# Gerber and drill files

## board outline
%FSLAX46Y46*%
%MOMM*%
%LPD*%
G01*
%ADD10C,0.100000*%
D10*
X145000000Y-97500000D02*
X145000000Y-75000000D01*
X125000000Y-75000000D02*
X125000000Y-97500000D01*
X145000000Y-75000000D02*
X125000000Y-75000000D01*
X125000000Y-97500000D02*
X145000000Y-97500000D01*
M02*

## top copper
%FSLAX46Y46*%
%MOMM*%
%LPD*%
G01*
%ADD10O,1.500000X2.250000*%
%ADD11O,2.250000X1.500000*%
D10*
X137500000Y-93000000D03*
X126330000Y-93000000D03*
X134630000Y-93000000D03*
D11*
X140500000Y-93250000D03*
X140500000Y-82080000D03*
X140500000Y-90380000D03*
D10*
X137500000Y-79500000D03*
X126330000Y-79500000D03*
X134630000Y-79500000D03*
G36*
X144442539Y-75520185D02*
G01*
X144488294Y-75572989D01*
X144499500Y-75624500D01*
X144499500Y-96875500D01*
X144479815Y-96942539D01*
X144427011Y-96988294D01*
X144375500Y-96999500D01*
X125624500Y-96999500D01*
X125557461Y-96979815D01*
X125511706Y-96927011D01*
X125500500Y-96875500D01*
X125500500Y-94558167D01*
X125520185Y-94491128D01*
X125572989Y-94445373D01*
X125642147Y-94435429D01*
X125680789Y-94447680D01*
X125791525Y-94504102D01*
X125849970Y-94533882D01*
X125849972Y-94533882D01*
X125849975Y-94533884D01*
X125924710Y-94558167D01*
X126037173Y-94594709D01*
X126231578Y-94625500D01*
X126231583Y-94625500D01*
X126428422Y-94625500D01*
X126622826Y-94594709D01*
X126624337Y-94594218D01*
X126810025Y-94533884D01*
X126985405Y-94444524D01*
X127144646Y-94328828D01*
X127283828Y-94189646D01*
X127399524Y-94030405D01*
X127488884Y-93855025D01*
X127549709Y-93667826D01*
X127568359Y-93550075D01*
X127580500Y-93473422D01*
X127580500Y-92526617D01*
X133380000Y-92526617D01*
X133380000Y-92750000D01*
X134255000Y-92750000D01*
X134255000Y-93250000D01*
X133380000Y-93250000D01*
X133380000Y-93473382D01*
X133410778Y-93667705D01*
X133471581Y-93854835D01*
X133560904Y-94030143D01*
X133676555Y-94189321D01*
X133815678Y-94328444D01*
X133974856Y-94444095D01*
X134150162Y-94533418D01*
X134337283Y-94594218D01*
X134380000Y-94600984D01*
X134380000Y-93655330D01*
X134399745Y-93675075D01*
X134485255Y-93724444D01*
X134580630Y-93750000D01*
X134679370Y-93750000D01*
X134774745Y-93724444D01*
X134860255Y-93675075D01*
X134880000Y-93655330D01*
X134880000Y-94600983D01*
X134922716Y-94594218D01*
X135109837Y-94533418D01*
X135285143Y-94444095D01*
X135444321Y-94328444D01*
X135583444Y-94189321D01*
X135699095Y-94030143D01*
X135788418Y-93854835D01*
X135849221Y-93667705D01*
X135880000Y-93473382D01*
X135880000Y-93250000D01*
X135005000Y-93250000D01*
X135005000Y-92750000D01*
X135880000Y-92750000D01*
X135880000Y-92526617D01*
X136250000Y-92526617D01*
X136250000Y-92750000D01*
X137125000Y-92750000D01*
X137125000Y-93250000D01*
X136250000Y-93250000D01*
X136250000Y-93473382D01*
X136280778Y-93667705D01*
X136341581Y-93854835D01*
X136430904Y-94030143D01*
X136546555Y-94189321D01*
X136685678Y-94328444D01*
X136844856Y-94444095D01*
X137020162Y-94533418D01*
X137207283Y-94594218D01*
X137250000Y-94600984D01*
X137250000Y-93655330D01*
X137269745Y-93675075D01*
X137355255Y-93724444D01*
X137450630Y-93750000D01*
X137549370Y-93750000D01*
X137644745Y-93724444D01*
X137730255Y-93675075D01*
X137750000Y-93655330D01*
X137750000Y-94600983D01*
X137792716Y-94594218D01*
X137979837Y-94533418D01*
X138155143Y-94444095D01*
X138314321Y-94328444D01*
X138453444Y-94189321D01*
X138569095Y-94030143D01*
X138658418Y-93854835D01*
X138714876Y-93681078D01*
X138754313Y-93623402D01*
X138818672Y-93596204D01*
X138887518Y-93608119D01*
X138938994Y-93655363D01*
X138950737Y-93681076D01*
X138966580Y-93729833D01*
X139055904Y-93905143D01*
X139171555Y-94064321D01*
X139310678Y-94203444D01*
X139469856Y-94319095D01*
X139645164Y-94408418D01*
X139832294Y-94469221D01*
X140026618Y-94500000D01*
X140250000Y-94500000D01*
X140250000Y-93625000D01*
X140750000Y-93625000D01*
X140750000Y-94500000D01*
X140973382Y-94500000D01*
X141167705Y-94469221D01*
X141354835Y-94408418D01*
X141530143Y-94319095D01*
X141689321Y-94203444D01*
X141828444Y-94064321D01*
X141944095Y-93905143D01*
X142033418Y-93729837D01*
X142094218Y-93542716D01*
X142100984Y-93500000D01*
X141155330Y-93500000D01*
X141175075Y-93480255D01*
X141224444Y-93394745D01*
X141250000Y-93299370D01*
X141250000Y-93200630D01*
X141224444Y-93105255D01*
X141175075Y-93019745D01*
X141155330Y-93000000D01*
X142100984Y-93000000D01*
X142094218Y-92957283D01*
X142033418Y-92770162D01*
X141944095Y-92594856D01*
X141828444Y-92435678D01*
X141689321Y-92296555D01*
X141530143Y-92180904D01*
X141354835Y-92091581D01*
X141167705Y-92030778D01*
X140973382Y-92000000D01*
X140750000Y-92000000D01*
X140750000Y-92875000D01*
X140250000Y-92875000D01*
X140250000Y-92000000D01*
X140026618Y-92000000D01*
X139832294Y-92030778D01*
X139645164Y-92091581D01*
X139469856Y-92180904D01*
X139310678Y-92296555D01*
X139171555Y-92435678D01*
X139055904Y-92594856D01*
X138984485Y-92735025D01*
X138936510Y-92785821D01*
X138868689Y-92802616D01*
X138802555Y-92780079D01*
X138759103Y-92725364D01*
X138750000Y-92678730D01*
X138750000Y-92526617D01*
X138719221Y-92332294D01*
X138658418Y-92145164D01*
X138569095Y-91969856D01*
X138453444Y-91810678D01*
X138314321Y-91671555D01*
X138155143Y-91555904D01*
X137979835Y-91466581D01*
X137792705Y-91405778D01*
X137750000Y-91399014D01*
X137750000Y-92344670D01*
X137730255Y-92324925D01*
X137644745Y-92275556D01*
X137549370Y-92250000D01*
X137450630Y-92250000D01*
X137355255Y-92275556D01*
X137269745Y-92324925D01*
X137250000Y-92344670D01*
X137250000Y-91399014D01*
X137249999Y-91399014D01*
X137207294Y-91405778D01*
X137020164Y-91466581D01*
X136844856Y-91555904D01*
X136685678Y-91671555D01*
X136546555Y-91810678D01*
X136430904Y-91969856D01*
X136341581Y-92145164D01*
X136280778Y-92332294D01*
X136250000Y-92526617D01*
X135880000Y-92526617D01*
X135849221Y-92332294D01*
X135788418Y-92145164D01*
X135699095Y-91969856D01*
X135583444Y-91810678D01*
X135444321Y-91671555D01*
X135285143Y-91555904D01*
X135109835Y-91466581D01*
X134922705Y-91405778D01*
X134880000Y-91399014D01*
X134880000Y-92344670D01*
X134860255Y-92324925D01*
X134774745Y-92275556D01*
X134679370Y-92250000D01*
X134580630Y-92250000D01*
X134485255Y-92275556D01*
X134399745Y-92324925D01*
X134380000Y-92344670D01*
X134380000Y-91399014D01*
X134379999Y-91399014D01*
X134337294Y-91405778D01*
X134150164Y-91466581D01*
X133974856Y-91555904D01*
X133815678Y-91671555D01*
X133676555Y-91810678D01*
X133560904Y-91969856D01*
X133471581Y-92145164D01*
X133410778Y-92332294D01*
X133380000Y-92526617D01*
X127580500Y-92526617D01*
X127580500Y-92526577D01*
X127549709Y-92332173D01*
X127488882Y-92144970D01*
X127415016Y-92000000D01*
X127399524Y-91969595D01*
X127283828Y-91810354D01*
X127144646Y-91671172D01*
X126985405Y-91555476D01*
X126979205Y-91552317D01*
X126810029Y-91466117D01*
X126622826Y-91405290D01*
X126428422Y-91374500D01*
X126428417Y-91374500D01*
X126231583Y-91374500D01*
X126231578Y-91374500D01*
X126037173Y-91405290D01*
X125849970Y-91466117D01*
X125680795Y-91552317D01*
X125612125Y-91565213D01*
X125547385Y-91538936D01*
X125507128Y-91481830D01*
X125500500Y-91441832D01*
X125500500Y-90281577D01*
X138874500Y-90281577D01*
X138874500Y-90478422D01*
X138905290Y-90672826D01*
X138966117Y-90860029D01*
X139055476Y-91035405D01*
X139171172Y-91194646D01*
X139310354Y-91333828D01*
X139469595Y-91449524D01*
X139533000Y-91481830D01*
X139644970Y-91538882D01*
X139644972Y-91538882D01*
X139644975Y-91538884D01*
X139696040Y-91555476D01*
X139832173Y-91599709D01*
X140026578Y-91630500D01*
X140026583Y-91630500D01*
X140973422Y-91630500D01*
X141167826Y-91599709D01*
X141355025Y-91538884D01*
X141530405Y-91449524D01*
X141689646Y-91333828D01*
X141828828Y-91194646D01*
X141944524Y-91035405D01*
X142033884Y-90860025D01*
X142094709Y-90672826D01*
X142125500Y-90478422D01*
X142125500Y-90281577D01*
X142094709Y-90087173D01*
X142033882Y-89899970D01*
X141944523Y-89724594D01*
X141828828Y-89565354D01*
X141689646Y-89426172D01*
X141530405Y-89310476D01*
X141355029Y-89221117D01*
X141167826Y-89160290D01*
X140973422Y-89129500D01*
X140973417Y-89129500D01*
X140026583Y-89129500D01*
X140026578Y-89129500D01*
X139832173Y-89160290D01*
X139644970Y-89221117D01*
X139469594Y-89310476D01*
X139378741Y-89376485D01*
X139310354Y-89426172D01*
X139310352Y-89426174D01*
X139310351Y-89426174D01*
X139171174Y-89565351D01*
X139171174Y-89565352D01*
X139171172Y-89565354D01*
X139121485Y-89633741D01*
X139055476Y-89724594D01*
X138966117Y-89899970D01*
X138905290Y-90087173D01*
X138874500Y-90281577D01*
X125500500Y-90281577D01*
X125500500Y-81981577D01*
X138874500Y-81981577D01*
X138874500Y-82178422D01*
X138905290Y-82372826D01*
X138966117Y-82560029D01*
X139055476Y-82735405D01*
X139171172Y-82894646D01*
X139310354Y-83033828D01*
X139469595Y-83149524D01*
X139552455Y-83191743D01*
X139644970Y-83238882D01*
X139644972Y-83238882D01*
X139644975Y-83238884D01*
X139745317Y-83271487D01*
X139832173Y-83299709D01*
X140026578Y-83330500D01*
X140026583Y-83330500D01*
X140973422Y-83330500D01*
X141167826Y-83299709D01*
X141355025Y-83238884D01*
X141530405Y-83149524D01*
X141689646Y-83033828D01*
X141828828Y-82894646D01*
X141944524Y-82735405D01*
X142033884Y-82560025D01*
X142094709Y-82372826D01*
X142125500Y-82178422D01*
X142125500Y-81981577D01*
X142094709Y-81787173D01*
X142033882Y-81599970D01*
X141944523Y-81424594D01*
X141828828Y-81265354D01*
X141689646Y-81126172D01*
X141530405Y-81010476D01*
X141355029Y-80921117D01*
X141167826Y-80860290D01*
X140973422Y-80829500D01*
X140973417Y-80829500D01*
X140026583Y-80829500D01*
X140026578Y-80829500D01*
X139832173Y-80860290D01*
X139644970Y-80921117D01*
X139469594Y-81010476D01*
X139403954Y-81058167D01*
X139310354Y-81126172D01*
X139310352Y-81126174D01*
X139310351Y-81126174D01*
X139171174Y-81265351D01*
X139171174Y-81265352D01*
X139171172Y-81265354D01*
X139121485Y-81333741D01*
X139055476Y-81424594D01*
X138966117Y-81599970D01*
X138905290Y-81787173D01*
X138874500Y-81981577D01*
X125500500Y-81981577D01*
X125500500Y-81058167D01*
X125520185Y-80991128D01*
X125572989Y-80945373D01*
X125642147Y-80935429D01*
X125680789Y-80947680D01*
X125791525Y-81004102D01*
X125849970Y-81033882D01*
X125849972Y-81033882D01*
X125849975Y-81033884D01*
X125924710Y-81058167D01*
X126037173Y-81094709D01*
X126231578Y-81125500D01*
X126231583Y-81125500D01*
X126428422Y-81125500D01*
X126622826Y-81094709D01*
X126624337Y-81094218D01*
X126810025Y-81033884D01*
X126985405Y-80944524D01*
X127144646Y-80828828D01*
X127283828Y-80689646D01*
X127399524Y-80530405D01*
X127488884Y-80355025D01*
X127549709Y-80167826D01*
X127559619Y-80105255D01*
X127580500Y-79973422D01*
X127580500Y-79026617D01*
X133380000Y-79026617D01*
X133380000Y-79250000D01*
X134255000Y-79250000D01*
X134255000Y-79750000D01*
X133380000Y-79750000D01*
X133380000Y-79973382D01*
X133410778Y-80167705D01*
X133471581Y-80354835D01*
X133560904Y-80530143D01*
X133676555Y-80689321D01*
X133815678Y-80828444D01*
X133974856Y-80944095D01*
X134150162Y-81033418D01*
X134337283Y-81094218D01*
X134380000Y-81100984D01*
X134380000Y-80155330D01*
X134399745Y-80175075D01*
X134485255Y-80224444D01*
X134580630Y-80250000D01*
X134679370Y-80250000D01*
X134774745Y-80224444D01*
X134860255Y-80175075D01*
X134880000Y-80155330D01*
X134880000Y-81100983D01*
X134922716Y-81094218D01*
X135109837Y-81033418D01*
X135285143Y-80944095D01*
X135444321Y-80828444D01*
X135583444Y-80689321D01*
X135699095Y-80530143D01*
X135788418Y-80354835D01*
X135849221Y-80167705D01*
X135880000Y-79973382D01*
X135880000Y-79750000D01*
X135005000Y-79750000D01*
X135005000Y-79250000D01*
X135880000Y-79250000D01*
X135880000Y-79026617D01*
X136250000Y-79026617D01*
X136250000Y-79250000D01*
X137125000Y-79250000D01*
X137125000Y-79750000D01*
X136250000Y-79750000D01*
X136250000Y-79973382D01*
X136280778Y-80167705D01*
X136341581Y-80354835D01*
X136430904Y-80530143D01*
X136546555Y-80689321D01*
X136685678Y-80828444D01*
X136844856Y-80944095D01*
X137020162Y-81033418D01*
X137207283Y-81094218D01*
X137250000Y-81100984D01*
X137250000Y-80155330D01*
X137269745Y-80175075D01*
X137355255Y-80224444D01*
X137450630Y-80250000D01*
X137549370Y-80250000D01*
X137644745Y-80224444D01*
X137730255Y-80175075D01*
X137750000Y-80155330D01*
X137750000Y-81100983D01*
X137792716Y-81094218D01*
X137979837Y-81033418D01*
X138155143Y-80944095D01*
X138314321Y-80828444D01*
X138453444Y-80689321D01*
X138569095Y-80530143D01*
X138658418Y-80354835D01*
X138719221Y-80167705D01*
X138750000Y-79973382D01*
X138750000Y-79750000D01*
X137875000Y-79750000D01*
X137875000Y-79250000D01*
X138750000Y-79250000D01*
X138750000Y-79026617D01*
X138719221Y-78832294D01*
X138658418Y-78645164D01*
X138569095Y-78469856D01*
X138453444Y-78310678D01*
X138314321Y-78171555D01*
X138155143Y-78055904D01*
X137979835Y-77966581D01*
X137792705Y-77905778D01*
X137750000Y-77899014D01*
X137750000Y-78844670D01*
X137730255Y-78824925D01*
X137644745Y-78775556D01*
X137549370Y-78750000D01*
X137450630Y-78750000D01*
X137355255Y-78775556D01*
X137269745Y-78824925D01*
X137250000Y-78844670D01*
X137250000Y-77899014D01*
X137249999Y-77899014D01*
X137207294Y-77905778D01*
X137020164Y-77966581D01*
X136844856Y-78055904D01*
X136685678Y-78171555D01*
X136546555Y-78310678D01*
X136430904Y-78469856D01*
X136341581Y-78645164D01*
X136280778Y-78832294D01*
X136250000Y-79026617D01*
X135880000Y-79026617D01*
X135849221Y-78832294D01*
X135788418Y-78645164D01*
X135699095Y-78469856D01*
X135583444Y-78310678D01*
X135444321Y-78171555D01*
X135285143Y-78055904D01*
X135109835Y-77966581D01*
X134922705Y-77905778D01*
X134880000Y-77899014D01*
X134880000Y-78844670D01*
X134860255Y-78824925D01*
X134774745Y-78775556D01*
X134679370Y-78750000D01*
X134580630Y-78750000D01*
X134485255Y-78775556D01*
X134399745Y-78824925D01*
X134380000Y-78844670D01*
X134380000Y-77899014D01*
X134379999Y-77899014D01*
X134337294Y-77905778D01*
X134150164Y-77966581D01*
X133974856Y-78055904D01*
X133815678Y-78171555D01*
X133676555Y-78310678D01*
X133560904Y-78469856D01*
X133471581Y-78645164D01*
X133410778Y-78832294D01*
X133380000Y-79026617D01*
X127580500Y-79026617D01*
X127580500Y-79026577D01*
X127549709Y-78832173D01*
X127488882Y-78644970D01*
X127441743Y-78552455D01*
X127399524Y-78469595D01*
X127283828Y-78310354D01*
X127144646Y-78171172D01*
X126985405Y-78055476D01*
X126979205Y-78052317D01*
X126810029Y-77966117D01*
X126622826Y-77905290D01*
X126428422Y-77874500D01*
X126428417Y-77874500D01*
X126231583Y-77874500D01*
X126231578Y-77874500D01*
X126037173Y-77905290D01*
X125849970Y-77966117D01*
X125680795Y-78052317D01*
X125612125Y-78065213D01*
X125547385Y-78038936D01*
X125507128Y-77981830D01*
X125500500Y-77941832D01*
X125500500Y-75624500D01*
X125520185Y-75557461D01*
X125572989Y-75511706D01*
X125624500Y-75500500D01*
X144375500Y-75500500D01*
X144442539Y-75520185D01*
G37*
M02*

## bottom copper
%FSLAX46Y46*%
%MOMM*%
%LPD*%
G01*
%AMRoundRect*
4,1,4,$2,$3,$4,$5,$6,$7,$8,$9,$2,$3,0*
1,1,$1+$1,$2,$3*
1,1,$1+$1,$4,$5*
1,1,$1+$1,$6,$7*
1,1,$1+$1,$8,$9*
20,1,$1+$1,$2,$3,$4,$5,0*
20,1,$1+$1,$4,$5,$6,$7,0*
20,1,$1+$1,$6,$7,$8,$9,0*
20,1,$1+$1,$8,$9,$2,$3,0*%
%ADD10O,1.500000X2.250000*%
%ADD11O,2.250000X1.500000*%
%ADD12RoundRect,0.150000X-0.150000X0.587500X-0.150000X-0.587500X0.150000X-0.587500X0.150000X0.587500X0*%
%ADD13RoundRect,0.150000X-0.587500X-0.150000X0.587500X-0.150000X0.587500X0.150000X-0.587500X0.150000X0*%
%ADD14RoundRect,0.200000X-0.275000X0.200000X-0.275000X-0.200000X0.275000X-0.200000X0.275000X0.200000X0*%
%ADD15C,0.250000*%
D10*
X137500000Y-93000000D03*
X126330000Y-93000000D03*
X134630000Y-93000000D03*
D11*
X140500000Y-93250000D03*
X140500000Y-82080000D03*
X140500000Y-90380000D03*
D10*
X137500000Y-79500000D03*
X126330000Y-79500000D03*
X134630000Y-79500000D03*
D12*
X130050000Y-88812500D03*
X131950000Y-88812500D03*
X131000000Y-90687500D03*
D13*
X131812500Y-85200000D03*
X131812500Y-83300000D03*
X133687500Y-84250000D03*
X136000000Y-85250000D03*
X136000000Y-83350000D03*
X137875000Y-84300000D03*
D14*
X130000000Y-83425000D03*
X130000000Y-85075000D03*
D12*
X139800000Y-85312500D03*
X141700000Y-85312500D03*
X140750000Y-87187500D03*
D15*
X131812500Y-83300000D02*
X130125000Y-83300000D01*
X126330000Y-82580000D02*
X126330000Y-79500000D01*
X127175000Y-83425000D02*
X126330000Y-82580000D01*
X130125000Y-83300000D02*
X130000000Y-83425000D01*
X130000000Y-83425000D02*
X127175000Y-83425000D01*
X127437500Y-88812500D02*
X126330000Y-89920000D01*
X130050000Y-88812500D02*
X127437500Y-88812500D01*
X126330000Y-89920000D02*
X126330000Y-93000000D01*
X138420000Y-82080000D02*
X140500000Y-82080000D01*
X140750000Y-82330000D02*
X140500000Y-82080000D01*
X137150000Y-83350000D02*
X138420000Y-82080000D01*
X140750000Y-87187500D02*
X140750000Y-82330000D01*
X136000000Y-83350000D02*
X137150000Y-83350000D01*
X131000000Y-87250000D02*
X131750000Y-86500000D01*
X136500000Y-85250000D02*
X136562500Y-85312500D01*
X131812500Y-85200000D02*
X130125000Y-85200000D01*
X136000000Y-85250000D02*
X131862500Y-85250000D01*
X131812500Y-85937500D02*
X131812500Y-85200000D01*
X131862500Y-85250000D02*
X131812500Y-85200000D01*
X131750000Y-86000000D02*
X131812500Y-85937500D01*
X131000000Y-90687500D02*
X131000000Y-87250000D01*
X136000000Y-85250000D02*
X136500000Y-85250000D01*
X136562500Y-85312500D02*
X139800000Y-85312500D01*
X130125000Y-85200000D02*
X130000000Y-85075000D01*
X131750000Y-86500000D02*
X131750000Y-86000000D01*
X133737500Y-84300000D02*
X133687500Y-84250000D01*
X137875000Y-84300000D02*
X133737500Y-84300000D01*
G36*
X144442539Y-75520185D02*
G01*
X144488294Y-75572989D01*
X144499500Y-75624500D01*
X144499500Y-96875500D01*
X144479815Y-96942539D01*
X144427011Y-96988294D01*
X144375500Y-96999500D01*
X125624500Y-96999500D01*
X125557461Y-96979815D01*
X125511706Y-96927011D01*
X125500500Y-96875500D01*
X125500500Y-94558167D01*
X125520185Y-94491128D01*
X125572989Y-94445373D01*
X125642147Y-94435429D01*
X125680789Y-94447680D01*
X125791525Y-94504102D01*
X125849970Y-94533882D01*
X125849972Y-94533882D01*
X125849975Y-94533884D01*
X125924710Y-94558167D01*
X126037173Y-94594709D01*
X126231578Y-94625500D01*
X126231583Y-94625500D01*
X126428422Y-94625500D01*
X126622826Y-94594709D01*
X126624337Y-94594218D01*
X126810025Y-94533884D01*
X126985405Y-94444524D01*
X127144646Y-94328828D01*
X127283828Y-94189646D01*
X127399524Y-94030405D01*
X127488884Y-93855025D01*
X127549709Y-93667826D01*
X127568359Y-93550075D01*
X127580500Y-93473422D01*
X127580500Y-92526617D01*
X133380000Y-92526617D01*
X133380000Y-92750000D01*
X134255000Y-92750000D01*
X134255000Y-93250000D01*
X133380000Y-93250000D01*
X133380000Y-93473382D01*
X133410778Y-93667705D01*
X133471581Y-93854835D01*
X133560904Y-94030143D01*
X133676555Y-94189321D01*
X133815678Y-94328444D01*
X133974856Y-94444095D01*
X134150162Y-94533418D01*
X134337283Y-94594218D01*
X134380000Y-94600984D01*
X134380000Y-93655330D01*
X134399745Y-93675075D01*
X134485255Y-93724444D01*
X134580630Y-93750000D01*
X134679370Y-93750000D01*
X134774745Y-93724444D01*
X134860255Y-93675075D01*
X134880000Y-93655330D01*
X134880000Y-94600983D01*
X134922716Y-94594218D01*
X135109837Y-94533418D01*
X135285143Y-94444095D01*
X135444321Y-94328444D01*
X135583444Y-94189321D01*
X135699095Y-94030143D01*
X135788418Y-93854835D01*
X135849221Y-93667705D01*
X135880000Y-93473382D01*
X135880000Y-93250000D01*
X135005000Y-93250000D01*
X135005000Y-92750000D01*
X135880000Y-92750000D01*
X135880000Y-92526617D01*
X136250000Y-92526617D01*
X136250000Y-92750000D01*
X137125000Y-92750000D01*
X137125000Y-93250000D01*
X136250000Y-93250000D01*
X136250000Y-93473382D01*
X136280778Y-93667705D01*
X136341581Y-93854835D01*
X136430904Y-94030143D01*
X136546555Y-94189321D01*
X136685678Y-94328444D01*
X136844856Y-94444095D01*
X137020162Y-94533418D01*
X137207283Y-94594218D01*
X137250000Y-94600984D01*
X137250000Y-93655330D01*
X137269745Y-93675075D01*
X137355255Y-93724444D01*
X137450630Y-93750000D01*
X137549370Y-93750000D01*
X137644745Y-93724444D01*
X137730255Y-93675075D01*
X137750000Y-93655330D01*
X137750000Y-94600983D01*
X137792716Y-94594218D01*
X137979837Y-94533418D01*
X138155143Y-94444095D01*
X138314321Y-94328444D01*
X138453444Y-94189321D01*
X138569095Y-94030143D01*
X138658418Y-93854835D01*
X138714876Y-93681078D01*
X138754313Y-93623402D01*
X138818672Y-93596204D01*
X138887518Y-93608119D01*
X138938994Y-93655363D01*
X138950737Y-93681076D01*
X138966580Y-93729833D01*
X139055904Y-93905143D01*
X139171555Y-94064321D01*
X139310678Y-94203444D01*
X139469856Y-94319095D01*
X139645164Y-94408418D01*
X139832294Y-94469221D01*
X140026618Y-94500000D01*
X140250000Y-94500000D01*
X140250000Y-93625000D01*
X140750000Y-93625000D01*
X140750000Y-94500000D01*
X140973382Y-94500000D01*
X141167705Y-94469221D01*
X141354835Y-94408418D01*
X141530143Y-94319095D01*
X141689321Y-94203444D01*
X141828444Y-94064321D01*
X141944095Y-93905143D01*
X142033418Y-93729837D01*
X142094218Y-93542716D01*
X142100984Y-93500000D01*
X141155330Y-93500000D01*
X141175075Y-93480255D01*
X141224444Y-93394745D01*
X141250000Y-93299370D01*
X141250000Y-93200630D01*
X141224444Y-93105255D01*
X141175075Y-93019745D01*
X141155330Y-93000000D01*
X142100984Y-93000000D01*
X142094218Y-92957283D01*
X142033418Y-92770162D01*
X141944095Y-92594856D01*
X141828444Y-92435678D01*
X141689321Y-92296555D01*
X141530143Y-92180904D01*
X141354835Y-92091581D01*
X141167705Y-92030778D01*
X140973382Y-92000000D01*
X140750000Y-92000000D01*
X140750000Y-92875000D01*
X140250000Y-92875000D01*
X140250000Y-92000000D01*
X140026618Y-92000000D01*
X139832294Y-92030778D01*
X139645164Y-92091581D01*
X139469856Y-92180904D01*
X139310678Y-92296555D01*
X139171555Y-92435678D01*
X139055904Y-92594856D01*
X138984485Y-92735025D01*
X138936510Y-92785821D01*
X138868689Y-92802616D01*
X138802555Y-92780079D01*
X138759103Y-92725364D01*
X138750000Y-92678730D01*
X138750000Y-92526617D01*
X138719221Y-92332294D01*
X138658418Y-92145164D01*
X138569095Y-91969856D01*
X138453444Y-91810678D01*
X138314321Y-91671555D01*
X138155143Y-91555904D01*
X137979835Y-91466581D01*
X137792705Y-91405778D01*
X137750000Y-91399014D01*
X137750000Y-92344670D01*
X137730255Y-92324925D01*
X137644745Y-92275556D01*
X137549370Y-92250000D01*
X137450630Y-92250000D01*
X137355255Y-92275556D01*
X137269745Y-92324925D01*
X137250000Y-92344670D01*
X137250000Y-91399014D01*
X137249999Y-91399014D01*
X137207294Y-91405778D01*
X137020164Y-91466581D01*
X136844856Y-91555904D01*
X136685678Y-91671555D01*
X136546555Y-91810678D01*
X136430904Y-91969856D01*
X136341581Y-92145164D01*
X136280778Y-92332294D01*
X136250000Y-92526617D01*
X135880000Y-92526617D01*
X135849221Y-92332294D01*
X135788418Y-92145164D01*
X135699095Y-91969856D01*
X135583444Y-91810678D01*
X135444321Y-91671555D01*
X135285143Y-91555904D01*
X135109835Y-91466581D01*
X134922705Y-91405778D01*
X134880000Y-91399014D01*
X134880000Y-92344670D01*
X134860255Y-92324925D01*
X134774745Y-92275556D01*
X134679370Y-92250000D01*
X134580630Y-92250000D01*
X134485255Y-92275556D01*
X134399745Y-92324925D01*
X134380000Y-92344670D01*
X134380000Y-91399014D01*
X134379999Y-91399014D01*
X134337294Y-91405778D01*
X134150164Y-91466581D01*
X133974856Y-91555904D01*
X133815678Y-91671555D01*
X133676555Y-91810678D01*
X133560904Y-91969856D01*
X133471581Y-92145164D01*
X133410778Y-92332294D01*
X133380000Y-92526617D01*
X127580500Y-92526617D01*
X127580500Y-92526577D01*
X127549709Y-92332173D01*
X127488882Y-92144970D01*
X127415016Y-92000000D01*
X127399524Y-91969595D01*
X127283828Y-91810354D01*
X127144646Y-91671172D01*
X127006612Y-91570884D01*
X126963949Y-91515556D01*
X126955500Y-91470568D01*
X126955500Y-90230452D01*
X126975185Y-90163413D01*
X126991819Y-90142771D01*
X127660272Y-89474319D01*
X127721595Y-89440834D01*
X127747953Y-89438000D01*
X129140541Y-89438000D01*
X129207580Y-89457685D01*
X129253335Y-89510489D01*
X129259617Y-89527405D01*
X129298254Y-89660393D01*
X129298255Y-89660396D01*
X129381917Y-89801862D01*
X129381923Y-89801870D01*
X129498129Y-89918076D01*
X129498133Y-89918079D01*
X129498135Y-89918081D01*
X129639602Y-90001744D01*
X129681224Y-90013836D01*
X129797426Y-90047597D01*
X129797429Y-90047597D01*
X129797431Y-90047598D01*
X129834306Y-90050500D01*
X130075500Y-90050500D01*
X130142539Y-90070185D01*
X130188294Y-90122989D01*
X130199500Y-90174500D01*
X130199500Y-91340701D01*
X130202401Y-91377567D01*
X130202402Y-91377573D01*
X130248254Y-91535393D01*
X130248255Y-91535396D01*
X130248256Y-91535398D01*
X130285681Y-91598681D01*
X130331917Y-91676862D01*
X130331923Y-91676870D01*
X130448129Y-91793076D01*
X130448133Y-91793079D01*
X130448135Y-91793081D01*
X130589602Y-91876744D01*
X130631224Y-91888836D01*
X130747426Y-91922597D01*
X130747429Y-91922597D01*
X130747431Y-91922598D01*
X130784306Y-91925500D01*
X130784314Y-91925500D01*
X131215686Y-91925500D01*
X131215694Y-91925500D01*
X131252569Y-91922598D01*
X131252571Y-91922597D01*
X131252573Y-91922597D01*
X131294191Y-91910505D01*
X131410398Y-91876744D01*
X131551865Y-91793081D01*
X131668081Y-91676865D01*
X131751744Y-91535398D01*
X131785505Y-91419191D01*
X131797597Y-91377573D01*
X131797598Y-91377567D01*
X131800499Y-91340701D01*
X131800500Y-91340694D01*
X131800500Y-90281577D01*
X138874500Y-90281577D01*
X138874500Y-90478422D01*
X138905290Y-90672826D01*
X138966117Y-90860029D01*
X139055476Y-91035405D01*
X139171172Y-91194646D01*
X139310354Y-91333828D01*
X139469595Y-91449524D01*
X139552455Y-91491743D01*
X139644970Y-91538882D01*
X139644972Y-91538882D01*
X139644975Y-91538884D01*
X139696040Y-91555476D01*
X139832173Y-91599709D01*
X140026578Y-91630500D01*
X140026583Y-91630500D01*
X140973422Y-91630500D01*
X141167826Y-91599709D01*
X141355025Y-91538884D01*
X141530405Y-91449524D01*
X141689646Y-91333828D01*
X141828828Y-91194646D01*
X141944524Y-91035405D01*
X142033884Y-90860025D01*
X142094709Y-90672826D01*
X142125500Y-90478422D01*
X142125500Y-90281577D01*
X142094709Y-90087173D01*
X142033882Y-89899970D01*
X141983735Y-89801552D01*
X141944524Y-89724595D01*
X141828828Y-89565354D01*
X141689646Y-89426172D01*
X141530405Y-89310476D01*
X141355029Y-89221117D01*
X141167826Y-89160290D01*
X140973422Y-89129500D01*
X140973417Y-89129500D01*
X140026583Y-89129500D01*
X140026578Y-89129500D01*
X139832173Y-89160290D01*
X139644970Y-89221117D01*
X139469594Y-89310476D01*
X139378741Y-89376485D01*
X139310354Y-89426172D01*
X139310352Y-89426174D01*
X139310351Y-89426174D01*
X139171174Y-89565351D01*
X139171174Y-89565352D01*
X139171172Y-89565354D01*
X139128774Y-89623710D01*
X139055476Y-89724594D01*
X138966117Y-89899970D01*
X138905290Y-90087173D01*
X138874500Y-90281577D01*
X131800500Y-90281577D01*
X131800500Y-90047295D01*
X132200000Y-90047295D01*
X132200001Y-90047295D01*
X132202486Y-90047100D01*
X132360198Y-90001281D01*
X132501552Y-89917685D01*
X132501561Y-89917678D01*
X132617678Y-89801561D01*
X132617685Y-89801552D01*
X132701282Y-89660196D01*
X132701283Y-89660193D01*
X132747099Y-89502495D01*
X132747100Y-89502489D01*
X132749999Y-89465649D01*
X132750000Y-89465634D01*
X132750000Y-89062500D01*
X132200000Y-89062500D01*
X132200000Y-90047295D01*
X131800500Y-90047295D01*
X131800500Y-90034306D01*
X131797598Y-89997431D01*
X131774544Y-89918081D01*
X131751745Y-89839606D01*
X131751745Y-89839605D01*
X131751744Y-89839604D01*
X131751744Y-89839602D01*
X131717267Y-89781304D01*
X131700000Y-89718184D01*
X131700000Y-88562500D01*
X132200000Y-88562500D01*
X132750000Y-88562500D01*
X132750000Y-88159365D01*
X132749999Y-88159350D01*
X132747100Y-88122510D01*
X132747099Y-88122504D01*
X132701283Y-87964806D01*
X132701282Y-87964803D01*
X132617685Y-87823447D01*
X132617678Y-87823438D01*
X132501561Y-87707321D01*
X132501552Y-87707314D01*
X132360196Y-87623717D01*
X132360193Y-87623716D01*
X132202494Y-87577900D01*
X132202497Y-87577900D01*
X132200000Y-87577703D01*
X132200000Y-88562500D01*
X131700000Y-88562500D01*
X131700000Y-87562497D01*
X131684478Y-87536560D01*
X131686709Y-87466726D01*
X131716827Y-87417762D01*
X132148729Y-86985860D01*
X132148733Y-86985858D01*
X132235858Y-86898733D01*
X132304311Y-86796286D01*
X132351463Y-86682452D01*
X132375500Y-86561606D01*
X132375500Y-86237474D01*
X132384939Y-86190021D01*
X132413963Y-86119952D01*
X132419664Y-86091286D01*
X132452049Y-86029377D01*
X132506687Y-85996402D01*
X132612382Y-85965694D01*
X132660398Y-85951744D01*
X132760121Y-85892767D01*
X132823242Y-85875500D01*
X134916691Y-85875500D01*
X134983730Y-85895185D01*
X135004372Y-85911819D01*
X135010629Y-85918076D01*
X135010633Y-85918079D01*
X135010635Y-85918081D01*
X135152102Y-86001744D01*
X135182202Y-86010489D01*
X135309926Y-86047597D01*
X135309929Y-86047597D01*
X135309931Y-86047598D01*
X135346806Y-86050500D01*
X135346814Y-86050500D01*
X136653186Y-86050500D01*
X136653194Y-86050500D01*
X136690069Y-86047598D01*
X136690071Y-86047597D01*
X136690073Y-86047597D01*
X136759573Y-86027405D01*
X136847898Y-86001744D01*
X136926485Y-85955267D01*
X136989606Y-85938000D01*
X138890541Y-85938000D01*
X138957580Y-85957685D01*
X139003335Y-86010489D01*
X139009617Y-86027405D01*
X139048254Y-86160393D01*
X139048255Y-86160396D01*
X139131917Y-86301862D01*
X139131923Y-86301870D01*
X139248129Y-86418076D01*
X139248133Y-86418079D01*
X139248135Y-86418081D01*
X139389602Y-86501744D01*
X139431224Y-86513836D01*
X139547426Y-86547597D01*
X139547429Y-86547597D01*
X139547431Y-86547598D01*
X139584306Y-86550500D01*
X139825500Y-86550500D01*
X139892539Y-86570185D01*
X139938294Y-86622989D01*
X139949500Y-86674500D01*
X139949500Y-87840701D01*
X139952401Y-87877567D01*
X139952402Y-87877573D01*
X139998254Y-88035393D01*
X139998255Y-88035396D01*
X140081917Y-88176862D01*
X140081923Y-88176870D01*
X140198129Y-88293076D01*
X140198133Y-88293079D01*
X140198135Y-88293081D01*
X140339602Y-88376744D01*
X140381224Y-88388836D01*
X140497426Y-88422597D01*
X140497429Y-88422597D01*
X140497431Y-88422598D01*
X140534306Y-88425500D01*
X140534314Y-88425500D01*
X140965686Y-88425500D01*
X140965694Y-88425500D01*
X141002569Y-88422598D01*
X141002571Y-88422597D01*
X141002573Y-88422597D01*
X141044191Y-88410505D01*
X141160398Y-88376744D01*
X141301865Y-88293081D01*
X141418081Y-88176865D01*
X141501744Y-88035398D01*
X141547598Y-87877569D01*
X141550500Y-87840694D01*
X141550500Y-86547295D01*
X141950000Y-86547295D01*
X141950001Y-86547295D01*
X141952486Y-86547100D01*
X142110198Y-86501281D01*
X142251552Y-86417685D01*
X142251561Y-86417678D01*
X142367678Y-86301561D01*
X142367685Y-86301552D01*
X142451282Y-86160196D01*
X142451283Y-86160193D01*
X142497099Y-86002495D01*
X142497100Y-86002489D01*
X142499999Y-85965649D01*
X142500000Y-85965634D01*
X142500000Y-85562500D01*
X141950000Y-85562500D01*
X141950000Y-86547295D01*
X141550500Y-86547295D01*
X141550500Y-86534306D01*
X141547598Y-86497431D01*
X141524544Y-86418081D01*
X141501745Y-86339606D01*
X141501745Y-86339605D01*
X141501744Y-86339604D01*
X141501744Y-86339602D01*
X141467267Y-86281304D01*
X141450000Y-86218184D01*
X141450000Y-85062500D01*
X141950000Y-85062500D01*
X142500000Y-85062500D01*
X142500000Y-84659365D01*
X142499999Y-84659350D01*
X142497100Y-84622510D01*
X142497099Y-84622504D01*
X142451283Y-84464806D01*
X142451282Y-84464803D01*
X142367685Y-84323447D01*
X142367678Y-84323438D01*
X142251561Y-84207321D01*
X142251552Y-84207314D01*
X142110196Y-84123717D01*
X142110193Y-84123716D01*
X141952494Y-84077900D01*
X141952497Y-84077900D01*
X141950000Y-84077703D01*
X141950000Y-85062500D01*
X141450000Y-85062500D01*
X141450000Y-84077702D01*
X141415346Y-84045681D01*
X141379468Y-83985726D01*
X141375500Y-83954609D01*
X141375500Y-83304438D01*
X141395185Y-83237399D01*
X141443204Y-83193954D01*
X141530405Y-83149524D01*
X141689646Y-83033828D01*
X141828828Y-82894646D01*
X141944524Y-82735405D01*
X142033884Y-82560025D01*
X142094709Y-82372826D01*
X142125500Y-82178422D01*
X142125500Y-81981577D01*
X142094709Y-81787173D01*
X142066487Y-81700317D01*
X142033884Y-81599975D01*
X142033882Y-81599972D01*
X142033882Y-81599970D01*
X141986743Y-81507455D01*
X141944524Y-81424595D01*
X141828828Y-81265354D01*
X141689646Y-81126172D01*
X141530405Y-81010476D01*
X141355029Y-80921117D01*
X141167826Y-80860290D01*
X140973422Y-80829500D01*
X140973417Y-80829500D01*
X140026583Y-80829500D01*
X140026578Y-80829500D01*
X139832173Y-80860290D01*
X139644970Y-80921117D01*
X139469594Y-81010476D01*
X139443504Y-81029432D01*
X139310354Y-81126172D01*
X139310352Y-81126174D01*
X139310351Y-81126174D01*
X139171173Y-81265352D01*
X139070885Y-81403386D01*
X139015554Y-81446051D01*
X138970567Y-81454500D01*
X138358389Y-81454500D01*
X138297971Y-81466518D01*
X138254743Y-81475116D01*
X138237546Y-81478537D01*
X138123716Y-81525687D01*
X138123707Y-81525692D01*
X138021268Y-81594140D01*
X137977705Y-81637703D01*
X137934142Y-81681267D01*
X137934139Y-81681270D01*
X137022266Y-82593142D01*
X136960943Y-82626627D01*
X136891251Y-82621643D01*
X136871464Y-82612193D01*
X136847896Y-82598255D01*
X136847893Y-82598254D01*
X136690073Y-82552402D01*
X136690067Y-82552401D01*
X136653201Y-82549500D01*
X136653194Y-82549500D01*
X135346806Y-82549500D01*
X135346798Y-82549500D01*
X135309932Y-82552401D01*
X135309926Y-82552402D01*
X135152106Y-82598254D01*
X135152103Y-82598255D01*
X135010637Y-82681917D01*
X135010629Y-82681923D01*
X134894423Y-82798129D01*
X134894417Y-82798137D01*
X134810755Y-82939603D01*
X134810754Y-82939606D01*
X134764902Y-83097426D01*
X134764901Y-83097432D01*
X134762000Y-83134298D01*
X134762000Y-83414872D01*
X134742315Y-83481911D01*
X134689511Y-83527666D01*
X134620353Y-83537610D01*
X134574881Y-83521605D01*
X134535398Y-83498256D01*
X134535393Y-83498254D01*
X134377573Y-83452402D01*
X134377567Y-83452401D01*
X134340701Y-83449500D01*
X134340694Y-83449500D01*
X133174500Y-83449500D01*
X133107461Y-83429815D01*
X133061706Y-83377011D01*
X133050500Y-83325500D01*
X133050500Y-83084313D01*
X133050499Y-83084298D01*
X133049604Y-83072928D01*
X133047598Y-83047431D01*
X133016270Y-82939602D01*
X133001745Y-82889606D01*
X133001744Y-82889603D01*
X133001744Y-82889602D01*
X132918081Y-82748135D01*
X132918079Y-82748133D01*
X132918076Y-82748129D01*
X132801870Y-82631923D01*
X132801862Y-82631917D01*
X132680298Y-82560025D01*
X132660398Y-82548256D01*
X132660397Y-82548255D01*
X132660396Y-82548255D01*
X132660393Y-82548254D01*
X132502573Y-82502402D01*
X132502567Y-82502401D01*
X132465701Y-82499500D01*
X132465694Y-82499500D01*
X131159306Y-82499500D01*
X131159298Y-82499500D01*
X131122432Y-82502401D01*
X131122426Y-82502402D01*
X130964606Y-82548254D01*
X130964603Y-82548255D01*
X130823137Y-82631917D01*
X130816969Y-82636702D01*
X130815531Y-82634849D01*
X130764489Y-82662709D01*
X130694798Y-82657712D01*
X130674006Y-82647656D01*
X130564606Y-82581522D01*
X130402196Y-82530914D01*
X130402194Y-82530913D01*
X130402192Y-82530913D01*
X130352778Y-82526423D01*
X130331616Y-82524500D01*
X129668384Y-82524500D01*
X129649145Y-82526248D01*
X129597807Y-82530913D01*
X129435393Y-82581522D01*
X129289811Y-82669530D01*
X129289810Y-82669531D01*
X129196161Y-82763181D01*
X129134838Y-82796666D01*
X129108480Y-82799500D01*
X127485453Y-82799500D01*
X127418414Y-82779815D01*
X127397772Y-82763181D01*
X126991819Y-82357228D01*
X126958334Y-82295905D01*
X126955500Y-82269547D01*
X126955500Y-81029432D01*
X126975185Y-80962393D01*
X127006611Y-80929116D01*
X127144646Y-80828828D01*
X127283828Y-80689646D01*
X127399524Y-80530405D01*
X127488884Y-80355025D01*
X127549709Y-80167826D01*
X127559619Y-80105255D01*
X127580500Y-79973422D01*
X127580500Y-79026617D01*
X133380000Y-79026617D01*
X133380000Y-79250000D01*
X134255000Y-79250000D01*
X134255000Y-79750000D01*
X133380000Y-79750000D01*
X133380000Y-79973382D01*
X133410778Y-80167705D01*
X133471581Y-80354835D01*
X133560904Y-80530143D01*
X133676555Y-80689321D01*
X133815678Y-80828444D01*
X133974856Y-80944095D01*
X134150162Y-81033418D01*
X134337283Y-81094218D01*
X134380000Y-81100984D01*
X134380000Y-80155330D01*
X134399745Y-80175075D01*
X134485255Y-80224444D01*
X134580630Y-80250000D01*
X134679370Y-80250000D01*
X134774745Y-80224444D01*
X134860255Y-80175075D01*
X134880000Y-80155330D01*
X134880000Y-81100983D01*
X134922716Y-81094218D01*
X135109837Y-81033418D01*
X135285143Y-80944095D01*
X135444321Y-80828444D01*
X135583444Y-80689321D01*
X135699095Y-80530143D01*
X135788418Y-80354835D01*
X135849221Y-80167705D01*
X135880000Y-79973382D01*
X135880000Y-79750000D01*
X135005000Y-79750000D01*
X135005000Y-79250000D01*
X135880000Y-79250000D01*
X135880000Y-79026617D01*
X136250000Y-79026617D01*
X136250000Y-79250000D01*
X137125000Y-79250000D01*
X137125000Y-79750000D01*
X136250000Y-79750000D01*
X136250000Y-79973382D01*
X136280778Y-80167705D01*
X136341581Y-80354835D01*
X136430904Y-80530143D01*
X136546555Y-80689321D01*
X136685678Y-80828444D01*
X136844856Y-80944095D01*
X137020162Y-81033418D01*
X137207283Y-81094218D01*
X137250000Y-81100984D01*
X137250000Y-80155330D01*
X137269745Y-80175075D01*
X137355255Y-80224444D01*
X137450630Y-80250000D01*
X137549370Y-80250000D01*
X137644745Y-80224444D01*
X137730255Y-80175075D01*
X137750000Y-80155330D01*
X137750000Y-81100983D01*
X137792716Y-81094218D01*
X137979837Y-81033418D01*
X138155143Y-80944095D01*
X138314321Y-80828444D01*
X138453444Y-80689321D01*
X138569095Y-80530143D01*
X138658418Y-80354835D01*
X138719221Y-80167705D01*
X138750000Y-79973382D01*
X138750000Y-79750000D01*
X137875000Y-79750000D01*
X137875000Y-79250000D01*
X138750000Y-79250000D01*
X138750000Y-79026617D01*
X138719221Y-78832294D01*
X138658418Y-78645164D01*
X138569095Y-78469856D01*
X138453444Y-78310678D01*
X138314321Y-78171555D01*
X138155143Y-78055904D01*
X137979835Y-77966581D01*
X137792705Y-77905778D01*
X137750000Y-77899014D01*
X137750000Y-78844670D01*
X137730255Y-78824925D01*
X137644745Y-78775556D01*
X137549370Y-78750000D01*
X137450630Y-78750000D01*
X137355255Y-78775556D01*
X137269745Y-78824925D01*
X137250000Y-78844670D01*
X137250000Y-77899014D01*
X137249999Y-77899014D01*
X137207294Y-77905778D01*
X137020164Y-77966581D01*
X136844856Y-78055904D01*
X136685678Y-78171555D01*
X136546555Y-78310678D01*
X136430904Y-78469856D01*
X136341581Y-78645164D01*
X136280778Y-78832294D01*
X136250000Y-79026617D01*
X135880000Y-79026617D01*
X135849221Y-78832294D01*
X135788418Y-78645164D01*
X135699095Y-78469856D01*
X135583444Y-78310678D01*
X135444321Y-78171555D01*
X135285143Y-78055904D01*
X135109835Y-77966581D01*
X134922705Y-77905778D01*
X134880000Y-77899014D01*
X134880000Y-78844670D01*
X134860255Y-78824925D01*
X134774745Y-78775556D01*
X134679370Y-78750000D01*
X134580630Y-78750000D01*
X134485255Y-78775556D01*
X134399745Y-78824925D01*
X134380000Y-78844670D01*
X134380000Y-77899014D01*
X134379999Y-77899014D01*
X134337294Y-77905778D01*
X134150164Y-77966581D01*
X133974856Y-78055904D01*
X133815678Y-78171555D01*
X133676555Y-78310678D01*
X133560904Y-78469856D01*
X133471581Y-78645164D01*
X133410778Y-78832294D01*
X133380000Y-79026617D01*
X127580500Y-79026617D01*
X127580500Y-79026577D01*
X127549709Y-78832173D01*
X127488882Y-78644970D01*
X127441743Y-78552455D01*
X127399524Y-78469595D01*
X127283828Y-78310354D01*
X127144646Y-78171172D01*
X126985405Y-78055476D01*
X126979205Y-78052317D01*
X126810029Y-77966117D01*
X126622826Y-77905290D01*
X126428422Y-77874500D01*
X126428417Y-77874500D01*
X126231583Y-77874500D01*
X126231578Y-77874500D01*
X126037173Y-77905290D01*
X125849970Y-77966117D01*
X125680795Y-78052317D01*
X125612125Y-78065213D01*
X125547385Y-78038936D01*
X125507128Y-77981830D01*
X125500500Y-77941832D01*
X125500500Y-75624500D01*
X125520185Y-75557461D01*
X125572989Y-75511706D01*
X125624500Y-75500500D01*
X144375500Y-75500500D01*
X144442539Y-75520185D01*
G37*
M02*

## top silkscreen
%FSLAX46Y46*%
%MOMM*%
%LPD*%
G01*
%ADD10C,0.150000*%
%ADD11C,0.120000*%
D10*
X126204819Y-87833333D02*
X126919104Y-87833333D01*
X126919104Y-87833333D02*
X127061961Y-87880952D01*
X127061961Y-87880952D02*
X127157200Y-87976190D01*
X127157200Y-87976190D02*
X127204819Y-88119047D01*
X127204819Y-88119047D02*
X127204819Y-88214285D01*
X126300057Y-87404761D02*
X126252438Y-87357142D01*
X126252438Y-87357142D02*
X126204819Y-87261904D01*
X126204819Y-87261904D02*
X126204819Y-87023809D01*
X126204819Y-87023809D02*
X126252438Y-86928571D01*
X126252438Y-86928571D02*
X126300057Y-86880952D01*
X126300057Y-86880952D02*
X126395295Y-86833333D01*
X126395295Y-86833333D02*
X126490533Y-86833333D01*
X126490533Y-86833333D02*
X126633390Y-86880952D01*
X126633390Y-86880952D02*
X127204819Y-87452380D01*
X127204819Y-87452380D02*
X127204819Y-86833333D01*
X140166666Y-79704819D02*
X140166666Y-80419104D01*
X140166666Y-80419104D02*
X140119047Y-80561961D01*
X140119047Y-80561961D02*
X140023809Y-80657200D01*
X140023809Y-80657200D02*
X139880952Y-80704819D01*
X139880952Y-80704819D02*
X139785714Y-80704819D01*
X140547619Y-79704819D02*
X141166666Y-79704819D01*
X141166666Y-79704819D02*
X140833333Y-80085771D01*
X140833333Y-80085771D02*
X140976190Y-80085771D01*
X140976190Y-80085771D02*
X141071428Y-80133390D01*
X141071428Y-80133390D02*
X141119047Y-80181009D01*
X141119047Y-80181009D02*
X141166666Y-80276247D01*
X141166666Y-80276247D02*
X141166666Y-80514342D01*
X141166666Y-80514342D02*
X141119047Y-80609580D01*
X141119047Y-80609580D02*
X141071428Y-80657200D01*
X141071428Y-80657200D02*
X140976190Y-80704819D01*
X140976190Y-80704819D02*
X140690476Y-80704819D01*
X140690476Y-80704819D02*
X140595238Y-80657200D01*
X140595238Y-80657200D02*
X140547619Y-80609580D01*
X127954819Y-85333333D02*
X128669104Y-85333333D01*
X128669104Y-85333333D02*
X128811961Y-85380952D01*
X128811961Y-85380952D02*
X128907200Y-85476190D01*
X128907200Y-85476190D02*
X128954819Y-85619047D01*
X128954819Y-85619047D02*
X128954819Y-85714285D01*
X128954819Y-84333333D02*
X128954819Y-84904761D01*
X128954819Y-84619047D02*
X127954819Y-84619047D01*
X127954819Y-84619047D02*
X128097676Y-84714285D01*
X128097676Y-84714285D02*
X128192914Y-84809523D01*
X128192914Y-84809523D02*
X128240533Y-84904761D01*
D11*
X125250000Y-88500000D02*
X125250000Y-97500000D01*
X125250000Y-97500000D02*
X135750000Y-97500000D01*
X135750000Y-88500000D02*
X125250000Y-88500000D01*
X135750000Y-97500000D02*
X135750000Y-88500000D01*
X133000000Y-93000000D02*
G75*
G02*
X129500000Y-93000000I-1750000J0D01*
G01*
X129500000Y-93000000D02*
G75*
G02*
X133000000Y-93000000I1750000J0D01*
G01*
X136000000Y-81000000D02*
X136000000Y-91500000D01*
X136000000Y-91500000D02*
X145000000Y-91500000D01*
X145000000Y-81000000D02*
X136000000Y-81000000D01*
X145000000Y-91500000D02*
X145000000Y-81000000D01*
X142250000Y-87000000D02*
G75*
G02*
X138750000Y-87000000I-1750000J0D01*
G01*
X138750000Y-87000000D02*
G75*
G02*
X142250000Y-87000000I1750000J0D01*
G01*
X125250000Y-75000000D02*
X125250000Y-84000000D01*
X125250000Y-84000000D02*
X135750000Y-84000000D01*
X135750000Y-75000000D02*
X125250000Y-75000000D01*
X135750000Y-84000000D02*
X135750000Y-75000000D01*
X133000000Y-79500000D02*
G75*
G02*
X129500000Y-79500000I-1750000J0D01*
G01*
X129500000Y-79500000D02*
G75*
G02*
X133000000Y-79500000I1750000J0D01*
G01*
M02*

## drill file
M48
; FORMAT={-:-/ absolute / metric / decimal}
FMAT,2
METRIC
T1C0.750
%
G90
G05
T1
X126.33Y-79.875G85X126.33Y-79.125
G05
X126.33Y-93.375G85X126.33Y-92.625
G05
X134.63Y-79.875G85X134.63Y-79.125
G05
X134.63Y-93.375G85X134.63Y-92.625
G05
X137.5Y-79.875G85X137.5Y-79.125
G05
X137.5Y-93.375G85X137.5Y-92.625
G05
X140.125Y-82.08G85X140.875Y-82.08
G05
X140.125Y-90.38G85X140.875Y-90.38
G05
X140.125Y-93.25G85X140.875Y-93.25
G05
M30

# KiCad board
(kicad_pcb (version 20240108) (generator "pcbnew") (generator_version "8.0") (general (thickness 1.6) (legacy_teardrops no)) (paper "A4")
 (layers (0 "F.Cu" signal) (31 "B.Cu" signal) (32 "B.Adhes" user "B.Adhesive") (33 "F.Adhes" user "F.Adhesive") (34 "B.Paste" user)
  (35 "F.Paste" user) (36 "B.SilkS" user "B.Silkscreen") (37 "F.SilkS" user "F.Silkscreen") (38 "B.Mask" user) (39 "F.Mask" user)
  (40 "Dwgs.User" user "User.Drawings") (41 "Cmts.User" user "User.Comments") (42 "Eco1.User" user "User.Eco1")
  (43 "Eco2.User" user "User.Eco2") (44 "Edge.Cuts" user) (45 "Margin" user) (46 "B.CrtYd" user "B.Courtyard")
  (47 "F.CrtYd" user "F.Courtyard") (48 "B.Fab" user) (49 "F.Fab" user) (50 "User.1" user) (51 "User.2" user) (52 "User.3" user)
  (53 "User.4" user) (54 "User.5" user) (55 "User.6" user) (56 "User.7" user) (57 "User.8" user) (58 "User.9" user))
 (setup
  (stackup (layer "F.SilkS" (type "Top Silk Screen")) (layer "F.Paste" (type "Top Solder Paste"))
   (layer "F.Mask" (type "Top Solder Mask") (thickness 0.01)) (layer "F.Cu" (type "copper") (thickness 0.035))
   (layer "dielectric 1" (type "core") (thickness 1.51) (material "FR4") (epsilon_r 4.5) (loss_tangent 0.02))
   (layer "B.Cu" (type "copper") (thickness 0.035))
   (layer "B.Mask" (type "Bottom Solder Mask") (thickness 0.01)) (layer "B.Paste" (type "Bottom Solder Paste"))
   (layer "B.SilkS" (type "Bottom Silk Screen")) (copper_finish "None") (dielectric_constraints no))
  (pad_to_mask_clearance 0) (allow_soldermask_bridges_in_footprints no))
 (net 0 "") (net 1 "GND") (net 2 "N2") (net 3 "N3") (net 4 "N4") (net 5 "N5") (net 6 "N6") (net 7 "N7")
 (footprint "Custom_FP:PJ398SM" (layer "F.Cu") (at 131.25 93 90)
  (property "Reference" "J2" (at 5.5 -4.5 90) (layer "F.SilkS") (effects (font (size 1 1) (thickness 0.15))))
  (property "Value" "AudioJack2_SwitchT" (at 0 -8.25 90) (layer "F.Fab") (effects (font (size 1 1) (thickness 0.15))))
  (fp_line (start 4.5 -6) (end -4.5 -6) (stroke (width 0.12) (type solid)) (layer "F.SilkS"))
  (fp_line (start -4.5 -6) (end -4.5 4.5) (stroke (width 0.12) (type solid)) (layer "F.SilkS"))
  (fp_line (start 4.5 4.5) (end 4.5 -6) (stroke (width 0.12) (type solid)) (layer "F.SilkS"))
  (fp_line (start -4.5 4.5) (end 4.5 4.5) (stroke (width 0.12) (type solid)) (layer "F.SilkS"))
  (fp_circle (center 0 0) (end 1.75 0) (stroke (width 0.12) (type solid)) (fill none) (layer "F.SilkS"))
  (pad "S" thru_hole oval (at 0 6.25 90) (size 2.25 1.5) (drill oval 1.5 0.75) (layers "*.Cu" "*.Mask") (remove_unused_layers no)
   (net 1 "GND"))
  (pad "T" thru_hole oval (at 0 -4.92 90) (size 2.25 1.5) (drill oval 1.5 0.75) (layers "*.Cu" "*.Mask") (remove_unused_layers no)
   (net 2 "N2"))
  (pad "TN" thru_hole oval (at 0 3.38 90) (size 2.25 1.5) (drill oval 1.5 0.75) (layers "*.Cu" "*.Mask") (remove_unused_layers no)
   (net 1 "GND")))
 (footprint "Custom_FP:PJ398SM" (layer "F.Cu") (at 140.5 87)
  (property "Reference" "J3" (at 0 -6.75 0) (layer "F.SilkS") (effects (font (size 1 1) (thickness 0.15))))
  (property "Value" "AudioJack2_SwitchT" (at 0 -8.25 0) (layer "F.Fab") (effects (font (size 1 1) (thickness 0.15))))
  (fp_line (start -4.5 -6) (end -4.5 4.5) (stroke (width 0.12) (type solid)) (layer "F.SilkS"))
  (fp_line (start -4.5 4.5) (end 4.5 4.5) (stroke (width 0.12) (type solid)) (layer "F.SilkS"))
  (fp_line (start 4.5 -6) (end -4.5 -6) (stroke (width 0.12) (type solid)) (layer "F.SilkS"))
  (fp_line (start 4.5 4.5) (end 4.5 -6) (stroke (width 0.12) (type solid)) (layer "F.SilkS"))
  (fp_circle (center 0 0) (end 1.75 0) (stroke (width 0.12) (type solid)) (fill none) (layer "F.SilkS"))
  (pad "S" thru_hole oval (at 0 6.25) (size 2.25 1.5) (drill oval 1.5 0.75) (layers "*.Cu" "*.Mask") (remove_unused_layers no) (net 1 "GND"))
  (pad "T" thru_hole oval (at 0 -4.92) (size 2.25 1.5) (drill oval 1.5 0.75) (layers "*.Cu" "*.Mask") (remove_unused_layers no) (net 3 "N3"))
  (pad "TN" thru_hole oval (at 0 3.38) (size 2.25 1.5) (drill oval 1.5 0.75) (layers "*.Cu" "*.Mask") (remove_unused_layers no) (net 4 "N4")))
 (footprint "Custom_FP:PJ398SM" (layer "F.Cu") (at 131.25 79.5 90)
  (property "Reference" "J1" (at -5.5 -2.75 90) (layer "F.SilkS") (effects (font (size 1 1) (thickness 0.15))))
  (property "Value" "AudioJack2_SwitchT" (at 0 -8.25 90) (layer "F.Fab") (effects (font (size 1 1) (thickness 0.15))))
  (fp_line (start 4.5 -6) (end -4.5 -6) (stroke (width 0.12) (type solid)) (layer "F.SilkS"))
  (fp_line (start -4.5 -6) (end -4.5 4.5) (stroke (width 0.12) (type solid)) (layer "F.SilkS"))
  (fp_line (start 4.5 4.5) (end 4.5 -6) (stroke (width 0.12) (type solid)) (layer "F.SilkS"))
  (fp_line (start -4.5 4.5) (end 4.5 4.5) (stroke (width 0.12) (type solid)) (layer "F.SilkS"))
  (fp_circle (center 0 0) (end 1.75 0) (stroke (width 0.12) (type solid)) (fill none) (layer "F.SilkS"))
  (pad "S" thru_hole oval (at 0 6.25 90) (size 2.25 1.5) (drill oval 1.5 0.75) (layers "*.Cu" "*.Mask") (remove_unused_layers no)
   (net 1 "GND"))
  (pad "T" thru_hole oval (at 0 -4.92 90) (size 2.25 1.5) (drill oval 1.5 0.75) (layers "*.Cu" "*.Mask") (remove_unused_layers no)
   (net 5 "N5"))
  (pad "TN" thru_hole oval (at 0 3.38 90) (size 2.25 1.5) (drill oval 1.5 0.75) (layers "*.Cu" "*.Mask") (remove_unused_layers no)
   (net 1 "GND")))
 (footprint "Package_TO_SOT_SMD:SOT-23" (layer "B.Cu") (at 131 89.75 -90)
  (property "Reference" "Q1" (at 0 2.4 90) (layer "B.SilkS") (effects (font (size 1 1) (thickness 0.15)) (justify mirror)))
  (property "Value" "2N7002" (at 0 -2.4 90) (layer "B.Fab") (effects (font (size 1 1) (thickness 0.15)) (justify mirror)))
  (pad "1" smd roundrect (at -0.9375 0.95 270) (size 1.475 0.6) (layers "B.Cu" "B.Paste" "B.Mask") (roundrect_rratio 0.25) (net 2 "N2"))
  (pad "2" smd roundrect (at -0.9375 -0.95 270) (size 1.475 0.6) (layers "B.Cu" "B.Paste" "B.Mask") (roundrect_rratio 0.25) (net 1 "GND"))
  (pad "3" smd roundrect (at 0.9375 0 270) (size 1.475 0.6) (layers "B.Cu" "B.Paste" "B.Mask") (roundrect_rratio 0.25) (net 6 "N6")))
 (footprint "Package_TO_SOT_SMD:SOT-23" (layer "B.Cu") (at 132.75 84.25)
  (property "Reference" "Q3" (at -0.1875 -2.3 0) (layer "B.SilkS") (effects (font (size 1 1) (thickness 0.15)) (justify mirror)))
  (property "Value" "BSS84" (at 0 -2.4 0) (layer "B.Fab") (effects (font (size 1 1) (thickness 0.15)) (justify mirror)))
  (pad "1" smd roundrect (at -0.9375 0.95) (size 1.475 0.6) (layers "B.Cu" "B.Paste" "B.Mask") (roundrect_rratio 0.25) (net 6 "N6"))
  (pad "2" smd roundrect (at -0.9375 -0.95) (size 1.475 0.6) (layers "B.Cu" "B.Paste" "B.Mask") (roundrect_rratio 0.25) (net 5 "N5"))
  (pad "3" smd roundrect (at 0.9375 0) (size 1.475 0.6) (layers "B.Cu" "B.Paste" "B.Mask") (roundrect_rratio 0.25) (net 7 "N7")))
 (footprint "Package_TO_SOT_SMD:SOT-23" (layer "B.Cu") (at 136.9375 84.3)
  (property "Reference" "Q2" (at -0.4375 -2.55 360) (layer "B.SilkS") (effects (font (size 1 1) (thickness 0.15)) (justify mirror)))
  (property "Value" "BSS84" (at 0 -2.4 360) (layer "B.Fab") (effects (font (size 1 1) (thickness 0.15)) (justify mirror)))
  (pad "1" smd roundrect (at -0.9375 0.95) (size 1.475 0.6) (layers "B.Cu" "B.Paste" "B.Mask") (roundrect_rratio 0.25) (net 6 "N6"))
  (pad "2" smd roundrect (at -0.9375 -0.95) (size 1.475 0.6) (layers "B.Cu" "B.Paste" "B.Mask") (roundrect_rratio 0.25) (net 3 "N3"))
  (pad "3" smd roundrect (at 0.9375 0) (size 1.475 0.6) (layers "B.Cu" "B.Paste" "B.Mask") (roundrect_rratio 0.25) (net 7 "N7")))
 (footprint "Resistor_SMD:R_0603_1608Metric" (layer "B.Cu") (at 130 84.25 -90)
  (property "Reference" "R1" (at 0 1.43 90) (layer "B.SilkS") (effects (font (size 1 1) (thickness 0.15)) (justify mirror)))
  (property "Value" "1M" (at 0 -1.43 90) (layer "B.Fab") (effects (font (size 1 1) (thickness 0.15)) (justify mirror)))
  (pad "1" smd roundrect (at -0.825 0 270) (size 0.8 0.95) (layers "B.Cu" "B.Paste" "B.Mask") (roundrect_rratio 0.25) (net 5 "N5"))
  (pad "2" smd roundrect (at 0.825 0 270) (size 0.8 0.95) (layers "B.Cu" "B.Paste" "B.Mask") (roundrect_rratio 0.25) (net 6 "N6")))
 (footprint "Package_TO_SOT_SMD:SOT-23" (layer "B.Cu") (at 140.75 86.25 -90)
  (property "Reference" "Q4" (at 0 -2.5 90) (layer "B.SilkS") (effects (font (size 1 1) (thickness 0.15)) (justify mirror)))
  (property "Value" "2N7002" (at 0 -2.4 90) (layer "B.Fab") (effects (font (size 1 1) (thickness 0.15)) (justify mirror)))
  (pad "1" smd roundrect (at -0.9375 0.95 270) (size 1.475 0.6) (layers "B.Cu" "B.Paste" "B.Mask") (roundrect_rratio 0.25) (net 6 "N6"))
  (pad "2" smd roundrect (at -0.9375 -0.95 270) (size 1.475 0.6) (layers "B.Cu" "B.Paste" "B.Mask") (roundrect_rratio 0.25) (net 1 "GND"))
  (pad "3" smd roundrect (at 0.9375 0 270) (size 1.475 0.6) (layers "B.Cu" "B.Paste" "B.Mask") (roundrect_rratio 0.25) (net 3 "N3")))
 (gr_line (start 145 97.5) (end 145 75) (stroke (width 0.1) (type default)) (layer "Edge.Cuts"))
 (gr_line (start 125 75) (end 125 97.5) (stroke (width 0.1) (type default)) (layer "Edge.Cuts"))
 (gr_line (start 145 75) (end 125 75) (stroke (width 0.1) (type default)) (layer "Edge.Cuts"))
 (gr_line (start 125 97.5) (end 145 97.5) (stroke (width 0.1) (type default)) (layer "Edge.Cuts"))
 (segment (start 131.8125 83.3) (end 130.125 83.3) (width 0.25) (layer "B.Cu") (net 5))
 (segment (start 126.33 82.58) (end 126.33 79.5) (width 0.25) (layer "B.Cu") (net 5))
 (segment (start 127.175 83.425) (end 126.33 82.58) (width 0.25) (layer "B.Cu") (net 5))
 (segment (start 130.125 83.3) (end 130 83.425) (width 0.25) (layer "B.Cu") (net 5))
 (segment (start 130 83.425) (end 127.175 83.425) (width 0.25) (layer "B.Cu") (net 5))
 (segment (start 127.4375 88.8125) (end 126.33 89.92) (width 0.25) (layer "B.Cu") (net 2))
 (segment (start 130.05 88.8125) (end 127.4375 88.8125) (width 0.25) (layer "B.Cu") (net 2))
 (segment (start 126.33 89.92) (end 126.33 93) (width 0.25) (layer "B.Cu") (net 2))
 (segment (start 138.42 82.08) (end 140.5 82.08) (width 0.25) (layer "B.Cu") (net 3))
 (segment (start 140.75 82.33) (end 140.5 82.08) (width 0.25) (layer "B.Cu") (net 3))
 (segment (start 137.15 83.35) (end 138.42 82.08) (width 0.25) (layer "B.Cu") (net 3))
 (segment (start 140.75 87.1875) (end 140.75 82.33) (width 0.25) (layer "B.Cu") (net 3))
 (segment (start 136 83.35) (end 137.15 83.35) (width 0.25) (layer "B.Cu") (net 3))
 (segment (start 131 87.25) (end 131.75 86.5) (width 0.25) (layer "B.Cu") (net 6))
 (segment (start 136.5 85.25) (end 136.5625 85.3125) (width 0.25) (layer "B.Cu") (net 6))
 (segment (start 131.8125 85.2) (end 130.125 85.2) (width 0.25) (layer "B.Cu") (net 6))
 (segment (start 136 85.25) (end 131.8625 85.25) (width 0.25) (layer "B.Cu") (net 6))
 (segment (start 131.8125 85.9375) (end 131.8125 85.2) (width 0.25) (layer "B.Cu") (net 6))
 (segment (start 131.8625 85.25) (end 131.8125 85.2) (width 0.25) (layer "B.Cu") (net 6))
 (segment (start 131.75 86) (end 131.8125 85.9375) (width 0.25) (layer "B.Cu") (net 6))
 (segment (start 131 90.6875) (end 131 87.25) (width 0.25) (layer "B.Cu") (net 6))
 (segment (start 136 85.25) (end 136.5 85.25) (width 0.25) (layer "B.Cu") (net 6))
 (segment (start 136.5625 85.3125) (end 139.8 85.3125) (width 0.25) (layer "B.Cu") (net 6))
 (segment (start 130.125 85.2) (end 130 85.075) (width 0.25) (layer "B.Cu") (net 6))
 (segment (start 131.75 86.5) (end 131.75 86) (width 0.25) (layer "B.Cu") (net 6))
 (segment (start 133.7375 84.3) (end 133.6875 84.25) (width 0.25) (layer "B.Cu") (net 7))
 (segment (start 137.875 84.3) (end 133.7375 84.3) (width 0.25) (layer "B.Cu") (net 7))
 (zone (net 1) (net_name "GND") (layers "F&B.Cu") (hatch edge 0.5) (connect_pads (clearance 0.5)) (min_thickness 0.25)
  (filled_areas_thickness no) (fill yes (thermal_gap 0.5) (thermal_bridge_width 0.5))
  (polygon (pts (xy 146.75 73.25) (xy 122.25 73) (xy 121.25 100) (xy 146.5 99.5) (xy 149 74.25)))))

